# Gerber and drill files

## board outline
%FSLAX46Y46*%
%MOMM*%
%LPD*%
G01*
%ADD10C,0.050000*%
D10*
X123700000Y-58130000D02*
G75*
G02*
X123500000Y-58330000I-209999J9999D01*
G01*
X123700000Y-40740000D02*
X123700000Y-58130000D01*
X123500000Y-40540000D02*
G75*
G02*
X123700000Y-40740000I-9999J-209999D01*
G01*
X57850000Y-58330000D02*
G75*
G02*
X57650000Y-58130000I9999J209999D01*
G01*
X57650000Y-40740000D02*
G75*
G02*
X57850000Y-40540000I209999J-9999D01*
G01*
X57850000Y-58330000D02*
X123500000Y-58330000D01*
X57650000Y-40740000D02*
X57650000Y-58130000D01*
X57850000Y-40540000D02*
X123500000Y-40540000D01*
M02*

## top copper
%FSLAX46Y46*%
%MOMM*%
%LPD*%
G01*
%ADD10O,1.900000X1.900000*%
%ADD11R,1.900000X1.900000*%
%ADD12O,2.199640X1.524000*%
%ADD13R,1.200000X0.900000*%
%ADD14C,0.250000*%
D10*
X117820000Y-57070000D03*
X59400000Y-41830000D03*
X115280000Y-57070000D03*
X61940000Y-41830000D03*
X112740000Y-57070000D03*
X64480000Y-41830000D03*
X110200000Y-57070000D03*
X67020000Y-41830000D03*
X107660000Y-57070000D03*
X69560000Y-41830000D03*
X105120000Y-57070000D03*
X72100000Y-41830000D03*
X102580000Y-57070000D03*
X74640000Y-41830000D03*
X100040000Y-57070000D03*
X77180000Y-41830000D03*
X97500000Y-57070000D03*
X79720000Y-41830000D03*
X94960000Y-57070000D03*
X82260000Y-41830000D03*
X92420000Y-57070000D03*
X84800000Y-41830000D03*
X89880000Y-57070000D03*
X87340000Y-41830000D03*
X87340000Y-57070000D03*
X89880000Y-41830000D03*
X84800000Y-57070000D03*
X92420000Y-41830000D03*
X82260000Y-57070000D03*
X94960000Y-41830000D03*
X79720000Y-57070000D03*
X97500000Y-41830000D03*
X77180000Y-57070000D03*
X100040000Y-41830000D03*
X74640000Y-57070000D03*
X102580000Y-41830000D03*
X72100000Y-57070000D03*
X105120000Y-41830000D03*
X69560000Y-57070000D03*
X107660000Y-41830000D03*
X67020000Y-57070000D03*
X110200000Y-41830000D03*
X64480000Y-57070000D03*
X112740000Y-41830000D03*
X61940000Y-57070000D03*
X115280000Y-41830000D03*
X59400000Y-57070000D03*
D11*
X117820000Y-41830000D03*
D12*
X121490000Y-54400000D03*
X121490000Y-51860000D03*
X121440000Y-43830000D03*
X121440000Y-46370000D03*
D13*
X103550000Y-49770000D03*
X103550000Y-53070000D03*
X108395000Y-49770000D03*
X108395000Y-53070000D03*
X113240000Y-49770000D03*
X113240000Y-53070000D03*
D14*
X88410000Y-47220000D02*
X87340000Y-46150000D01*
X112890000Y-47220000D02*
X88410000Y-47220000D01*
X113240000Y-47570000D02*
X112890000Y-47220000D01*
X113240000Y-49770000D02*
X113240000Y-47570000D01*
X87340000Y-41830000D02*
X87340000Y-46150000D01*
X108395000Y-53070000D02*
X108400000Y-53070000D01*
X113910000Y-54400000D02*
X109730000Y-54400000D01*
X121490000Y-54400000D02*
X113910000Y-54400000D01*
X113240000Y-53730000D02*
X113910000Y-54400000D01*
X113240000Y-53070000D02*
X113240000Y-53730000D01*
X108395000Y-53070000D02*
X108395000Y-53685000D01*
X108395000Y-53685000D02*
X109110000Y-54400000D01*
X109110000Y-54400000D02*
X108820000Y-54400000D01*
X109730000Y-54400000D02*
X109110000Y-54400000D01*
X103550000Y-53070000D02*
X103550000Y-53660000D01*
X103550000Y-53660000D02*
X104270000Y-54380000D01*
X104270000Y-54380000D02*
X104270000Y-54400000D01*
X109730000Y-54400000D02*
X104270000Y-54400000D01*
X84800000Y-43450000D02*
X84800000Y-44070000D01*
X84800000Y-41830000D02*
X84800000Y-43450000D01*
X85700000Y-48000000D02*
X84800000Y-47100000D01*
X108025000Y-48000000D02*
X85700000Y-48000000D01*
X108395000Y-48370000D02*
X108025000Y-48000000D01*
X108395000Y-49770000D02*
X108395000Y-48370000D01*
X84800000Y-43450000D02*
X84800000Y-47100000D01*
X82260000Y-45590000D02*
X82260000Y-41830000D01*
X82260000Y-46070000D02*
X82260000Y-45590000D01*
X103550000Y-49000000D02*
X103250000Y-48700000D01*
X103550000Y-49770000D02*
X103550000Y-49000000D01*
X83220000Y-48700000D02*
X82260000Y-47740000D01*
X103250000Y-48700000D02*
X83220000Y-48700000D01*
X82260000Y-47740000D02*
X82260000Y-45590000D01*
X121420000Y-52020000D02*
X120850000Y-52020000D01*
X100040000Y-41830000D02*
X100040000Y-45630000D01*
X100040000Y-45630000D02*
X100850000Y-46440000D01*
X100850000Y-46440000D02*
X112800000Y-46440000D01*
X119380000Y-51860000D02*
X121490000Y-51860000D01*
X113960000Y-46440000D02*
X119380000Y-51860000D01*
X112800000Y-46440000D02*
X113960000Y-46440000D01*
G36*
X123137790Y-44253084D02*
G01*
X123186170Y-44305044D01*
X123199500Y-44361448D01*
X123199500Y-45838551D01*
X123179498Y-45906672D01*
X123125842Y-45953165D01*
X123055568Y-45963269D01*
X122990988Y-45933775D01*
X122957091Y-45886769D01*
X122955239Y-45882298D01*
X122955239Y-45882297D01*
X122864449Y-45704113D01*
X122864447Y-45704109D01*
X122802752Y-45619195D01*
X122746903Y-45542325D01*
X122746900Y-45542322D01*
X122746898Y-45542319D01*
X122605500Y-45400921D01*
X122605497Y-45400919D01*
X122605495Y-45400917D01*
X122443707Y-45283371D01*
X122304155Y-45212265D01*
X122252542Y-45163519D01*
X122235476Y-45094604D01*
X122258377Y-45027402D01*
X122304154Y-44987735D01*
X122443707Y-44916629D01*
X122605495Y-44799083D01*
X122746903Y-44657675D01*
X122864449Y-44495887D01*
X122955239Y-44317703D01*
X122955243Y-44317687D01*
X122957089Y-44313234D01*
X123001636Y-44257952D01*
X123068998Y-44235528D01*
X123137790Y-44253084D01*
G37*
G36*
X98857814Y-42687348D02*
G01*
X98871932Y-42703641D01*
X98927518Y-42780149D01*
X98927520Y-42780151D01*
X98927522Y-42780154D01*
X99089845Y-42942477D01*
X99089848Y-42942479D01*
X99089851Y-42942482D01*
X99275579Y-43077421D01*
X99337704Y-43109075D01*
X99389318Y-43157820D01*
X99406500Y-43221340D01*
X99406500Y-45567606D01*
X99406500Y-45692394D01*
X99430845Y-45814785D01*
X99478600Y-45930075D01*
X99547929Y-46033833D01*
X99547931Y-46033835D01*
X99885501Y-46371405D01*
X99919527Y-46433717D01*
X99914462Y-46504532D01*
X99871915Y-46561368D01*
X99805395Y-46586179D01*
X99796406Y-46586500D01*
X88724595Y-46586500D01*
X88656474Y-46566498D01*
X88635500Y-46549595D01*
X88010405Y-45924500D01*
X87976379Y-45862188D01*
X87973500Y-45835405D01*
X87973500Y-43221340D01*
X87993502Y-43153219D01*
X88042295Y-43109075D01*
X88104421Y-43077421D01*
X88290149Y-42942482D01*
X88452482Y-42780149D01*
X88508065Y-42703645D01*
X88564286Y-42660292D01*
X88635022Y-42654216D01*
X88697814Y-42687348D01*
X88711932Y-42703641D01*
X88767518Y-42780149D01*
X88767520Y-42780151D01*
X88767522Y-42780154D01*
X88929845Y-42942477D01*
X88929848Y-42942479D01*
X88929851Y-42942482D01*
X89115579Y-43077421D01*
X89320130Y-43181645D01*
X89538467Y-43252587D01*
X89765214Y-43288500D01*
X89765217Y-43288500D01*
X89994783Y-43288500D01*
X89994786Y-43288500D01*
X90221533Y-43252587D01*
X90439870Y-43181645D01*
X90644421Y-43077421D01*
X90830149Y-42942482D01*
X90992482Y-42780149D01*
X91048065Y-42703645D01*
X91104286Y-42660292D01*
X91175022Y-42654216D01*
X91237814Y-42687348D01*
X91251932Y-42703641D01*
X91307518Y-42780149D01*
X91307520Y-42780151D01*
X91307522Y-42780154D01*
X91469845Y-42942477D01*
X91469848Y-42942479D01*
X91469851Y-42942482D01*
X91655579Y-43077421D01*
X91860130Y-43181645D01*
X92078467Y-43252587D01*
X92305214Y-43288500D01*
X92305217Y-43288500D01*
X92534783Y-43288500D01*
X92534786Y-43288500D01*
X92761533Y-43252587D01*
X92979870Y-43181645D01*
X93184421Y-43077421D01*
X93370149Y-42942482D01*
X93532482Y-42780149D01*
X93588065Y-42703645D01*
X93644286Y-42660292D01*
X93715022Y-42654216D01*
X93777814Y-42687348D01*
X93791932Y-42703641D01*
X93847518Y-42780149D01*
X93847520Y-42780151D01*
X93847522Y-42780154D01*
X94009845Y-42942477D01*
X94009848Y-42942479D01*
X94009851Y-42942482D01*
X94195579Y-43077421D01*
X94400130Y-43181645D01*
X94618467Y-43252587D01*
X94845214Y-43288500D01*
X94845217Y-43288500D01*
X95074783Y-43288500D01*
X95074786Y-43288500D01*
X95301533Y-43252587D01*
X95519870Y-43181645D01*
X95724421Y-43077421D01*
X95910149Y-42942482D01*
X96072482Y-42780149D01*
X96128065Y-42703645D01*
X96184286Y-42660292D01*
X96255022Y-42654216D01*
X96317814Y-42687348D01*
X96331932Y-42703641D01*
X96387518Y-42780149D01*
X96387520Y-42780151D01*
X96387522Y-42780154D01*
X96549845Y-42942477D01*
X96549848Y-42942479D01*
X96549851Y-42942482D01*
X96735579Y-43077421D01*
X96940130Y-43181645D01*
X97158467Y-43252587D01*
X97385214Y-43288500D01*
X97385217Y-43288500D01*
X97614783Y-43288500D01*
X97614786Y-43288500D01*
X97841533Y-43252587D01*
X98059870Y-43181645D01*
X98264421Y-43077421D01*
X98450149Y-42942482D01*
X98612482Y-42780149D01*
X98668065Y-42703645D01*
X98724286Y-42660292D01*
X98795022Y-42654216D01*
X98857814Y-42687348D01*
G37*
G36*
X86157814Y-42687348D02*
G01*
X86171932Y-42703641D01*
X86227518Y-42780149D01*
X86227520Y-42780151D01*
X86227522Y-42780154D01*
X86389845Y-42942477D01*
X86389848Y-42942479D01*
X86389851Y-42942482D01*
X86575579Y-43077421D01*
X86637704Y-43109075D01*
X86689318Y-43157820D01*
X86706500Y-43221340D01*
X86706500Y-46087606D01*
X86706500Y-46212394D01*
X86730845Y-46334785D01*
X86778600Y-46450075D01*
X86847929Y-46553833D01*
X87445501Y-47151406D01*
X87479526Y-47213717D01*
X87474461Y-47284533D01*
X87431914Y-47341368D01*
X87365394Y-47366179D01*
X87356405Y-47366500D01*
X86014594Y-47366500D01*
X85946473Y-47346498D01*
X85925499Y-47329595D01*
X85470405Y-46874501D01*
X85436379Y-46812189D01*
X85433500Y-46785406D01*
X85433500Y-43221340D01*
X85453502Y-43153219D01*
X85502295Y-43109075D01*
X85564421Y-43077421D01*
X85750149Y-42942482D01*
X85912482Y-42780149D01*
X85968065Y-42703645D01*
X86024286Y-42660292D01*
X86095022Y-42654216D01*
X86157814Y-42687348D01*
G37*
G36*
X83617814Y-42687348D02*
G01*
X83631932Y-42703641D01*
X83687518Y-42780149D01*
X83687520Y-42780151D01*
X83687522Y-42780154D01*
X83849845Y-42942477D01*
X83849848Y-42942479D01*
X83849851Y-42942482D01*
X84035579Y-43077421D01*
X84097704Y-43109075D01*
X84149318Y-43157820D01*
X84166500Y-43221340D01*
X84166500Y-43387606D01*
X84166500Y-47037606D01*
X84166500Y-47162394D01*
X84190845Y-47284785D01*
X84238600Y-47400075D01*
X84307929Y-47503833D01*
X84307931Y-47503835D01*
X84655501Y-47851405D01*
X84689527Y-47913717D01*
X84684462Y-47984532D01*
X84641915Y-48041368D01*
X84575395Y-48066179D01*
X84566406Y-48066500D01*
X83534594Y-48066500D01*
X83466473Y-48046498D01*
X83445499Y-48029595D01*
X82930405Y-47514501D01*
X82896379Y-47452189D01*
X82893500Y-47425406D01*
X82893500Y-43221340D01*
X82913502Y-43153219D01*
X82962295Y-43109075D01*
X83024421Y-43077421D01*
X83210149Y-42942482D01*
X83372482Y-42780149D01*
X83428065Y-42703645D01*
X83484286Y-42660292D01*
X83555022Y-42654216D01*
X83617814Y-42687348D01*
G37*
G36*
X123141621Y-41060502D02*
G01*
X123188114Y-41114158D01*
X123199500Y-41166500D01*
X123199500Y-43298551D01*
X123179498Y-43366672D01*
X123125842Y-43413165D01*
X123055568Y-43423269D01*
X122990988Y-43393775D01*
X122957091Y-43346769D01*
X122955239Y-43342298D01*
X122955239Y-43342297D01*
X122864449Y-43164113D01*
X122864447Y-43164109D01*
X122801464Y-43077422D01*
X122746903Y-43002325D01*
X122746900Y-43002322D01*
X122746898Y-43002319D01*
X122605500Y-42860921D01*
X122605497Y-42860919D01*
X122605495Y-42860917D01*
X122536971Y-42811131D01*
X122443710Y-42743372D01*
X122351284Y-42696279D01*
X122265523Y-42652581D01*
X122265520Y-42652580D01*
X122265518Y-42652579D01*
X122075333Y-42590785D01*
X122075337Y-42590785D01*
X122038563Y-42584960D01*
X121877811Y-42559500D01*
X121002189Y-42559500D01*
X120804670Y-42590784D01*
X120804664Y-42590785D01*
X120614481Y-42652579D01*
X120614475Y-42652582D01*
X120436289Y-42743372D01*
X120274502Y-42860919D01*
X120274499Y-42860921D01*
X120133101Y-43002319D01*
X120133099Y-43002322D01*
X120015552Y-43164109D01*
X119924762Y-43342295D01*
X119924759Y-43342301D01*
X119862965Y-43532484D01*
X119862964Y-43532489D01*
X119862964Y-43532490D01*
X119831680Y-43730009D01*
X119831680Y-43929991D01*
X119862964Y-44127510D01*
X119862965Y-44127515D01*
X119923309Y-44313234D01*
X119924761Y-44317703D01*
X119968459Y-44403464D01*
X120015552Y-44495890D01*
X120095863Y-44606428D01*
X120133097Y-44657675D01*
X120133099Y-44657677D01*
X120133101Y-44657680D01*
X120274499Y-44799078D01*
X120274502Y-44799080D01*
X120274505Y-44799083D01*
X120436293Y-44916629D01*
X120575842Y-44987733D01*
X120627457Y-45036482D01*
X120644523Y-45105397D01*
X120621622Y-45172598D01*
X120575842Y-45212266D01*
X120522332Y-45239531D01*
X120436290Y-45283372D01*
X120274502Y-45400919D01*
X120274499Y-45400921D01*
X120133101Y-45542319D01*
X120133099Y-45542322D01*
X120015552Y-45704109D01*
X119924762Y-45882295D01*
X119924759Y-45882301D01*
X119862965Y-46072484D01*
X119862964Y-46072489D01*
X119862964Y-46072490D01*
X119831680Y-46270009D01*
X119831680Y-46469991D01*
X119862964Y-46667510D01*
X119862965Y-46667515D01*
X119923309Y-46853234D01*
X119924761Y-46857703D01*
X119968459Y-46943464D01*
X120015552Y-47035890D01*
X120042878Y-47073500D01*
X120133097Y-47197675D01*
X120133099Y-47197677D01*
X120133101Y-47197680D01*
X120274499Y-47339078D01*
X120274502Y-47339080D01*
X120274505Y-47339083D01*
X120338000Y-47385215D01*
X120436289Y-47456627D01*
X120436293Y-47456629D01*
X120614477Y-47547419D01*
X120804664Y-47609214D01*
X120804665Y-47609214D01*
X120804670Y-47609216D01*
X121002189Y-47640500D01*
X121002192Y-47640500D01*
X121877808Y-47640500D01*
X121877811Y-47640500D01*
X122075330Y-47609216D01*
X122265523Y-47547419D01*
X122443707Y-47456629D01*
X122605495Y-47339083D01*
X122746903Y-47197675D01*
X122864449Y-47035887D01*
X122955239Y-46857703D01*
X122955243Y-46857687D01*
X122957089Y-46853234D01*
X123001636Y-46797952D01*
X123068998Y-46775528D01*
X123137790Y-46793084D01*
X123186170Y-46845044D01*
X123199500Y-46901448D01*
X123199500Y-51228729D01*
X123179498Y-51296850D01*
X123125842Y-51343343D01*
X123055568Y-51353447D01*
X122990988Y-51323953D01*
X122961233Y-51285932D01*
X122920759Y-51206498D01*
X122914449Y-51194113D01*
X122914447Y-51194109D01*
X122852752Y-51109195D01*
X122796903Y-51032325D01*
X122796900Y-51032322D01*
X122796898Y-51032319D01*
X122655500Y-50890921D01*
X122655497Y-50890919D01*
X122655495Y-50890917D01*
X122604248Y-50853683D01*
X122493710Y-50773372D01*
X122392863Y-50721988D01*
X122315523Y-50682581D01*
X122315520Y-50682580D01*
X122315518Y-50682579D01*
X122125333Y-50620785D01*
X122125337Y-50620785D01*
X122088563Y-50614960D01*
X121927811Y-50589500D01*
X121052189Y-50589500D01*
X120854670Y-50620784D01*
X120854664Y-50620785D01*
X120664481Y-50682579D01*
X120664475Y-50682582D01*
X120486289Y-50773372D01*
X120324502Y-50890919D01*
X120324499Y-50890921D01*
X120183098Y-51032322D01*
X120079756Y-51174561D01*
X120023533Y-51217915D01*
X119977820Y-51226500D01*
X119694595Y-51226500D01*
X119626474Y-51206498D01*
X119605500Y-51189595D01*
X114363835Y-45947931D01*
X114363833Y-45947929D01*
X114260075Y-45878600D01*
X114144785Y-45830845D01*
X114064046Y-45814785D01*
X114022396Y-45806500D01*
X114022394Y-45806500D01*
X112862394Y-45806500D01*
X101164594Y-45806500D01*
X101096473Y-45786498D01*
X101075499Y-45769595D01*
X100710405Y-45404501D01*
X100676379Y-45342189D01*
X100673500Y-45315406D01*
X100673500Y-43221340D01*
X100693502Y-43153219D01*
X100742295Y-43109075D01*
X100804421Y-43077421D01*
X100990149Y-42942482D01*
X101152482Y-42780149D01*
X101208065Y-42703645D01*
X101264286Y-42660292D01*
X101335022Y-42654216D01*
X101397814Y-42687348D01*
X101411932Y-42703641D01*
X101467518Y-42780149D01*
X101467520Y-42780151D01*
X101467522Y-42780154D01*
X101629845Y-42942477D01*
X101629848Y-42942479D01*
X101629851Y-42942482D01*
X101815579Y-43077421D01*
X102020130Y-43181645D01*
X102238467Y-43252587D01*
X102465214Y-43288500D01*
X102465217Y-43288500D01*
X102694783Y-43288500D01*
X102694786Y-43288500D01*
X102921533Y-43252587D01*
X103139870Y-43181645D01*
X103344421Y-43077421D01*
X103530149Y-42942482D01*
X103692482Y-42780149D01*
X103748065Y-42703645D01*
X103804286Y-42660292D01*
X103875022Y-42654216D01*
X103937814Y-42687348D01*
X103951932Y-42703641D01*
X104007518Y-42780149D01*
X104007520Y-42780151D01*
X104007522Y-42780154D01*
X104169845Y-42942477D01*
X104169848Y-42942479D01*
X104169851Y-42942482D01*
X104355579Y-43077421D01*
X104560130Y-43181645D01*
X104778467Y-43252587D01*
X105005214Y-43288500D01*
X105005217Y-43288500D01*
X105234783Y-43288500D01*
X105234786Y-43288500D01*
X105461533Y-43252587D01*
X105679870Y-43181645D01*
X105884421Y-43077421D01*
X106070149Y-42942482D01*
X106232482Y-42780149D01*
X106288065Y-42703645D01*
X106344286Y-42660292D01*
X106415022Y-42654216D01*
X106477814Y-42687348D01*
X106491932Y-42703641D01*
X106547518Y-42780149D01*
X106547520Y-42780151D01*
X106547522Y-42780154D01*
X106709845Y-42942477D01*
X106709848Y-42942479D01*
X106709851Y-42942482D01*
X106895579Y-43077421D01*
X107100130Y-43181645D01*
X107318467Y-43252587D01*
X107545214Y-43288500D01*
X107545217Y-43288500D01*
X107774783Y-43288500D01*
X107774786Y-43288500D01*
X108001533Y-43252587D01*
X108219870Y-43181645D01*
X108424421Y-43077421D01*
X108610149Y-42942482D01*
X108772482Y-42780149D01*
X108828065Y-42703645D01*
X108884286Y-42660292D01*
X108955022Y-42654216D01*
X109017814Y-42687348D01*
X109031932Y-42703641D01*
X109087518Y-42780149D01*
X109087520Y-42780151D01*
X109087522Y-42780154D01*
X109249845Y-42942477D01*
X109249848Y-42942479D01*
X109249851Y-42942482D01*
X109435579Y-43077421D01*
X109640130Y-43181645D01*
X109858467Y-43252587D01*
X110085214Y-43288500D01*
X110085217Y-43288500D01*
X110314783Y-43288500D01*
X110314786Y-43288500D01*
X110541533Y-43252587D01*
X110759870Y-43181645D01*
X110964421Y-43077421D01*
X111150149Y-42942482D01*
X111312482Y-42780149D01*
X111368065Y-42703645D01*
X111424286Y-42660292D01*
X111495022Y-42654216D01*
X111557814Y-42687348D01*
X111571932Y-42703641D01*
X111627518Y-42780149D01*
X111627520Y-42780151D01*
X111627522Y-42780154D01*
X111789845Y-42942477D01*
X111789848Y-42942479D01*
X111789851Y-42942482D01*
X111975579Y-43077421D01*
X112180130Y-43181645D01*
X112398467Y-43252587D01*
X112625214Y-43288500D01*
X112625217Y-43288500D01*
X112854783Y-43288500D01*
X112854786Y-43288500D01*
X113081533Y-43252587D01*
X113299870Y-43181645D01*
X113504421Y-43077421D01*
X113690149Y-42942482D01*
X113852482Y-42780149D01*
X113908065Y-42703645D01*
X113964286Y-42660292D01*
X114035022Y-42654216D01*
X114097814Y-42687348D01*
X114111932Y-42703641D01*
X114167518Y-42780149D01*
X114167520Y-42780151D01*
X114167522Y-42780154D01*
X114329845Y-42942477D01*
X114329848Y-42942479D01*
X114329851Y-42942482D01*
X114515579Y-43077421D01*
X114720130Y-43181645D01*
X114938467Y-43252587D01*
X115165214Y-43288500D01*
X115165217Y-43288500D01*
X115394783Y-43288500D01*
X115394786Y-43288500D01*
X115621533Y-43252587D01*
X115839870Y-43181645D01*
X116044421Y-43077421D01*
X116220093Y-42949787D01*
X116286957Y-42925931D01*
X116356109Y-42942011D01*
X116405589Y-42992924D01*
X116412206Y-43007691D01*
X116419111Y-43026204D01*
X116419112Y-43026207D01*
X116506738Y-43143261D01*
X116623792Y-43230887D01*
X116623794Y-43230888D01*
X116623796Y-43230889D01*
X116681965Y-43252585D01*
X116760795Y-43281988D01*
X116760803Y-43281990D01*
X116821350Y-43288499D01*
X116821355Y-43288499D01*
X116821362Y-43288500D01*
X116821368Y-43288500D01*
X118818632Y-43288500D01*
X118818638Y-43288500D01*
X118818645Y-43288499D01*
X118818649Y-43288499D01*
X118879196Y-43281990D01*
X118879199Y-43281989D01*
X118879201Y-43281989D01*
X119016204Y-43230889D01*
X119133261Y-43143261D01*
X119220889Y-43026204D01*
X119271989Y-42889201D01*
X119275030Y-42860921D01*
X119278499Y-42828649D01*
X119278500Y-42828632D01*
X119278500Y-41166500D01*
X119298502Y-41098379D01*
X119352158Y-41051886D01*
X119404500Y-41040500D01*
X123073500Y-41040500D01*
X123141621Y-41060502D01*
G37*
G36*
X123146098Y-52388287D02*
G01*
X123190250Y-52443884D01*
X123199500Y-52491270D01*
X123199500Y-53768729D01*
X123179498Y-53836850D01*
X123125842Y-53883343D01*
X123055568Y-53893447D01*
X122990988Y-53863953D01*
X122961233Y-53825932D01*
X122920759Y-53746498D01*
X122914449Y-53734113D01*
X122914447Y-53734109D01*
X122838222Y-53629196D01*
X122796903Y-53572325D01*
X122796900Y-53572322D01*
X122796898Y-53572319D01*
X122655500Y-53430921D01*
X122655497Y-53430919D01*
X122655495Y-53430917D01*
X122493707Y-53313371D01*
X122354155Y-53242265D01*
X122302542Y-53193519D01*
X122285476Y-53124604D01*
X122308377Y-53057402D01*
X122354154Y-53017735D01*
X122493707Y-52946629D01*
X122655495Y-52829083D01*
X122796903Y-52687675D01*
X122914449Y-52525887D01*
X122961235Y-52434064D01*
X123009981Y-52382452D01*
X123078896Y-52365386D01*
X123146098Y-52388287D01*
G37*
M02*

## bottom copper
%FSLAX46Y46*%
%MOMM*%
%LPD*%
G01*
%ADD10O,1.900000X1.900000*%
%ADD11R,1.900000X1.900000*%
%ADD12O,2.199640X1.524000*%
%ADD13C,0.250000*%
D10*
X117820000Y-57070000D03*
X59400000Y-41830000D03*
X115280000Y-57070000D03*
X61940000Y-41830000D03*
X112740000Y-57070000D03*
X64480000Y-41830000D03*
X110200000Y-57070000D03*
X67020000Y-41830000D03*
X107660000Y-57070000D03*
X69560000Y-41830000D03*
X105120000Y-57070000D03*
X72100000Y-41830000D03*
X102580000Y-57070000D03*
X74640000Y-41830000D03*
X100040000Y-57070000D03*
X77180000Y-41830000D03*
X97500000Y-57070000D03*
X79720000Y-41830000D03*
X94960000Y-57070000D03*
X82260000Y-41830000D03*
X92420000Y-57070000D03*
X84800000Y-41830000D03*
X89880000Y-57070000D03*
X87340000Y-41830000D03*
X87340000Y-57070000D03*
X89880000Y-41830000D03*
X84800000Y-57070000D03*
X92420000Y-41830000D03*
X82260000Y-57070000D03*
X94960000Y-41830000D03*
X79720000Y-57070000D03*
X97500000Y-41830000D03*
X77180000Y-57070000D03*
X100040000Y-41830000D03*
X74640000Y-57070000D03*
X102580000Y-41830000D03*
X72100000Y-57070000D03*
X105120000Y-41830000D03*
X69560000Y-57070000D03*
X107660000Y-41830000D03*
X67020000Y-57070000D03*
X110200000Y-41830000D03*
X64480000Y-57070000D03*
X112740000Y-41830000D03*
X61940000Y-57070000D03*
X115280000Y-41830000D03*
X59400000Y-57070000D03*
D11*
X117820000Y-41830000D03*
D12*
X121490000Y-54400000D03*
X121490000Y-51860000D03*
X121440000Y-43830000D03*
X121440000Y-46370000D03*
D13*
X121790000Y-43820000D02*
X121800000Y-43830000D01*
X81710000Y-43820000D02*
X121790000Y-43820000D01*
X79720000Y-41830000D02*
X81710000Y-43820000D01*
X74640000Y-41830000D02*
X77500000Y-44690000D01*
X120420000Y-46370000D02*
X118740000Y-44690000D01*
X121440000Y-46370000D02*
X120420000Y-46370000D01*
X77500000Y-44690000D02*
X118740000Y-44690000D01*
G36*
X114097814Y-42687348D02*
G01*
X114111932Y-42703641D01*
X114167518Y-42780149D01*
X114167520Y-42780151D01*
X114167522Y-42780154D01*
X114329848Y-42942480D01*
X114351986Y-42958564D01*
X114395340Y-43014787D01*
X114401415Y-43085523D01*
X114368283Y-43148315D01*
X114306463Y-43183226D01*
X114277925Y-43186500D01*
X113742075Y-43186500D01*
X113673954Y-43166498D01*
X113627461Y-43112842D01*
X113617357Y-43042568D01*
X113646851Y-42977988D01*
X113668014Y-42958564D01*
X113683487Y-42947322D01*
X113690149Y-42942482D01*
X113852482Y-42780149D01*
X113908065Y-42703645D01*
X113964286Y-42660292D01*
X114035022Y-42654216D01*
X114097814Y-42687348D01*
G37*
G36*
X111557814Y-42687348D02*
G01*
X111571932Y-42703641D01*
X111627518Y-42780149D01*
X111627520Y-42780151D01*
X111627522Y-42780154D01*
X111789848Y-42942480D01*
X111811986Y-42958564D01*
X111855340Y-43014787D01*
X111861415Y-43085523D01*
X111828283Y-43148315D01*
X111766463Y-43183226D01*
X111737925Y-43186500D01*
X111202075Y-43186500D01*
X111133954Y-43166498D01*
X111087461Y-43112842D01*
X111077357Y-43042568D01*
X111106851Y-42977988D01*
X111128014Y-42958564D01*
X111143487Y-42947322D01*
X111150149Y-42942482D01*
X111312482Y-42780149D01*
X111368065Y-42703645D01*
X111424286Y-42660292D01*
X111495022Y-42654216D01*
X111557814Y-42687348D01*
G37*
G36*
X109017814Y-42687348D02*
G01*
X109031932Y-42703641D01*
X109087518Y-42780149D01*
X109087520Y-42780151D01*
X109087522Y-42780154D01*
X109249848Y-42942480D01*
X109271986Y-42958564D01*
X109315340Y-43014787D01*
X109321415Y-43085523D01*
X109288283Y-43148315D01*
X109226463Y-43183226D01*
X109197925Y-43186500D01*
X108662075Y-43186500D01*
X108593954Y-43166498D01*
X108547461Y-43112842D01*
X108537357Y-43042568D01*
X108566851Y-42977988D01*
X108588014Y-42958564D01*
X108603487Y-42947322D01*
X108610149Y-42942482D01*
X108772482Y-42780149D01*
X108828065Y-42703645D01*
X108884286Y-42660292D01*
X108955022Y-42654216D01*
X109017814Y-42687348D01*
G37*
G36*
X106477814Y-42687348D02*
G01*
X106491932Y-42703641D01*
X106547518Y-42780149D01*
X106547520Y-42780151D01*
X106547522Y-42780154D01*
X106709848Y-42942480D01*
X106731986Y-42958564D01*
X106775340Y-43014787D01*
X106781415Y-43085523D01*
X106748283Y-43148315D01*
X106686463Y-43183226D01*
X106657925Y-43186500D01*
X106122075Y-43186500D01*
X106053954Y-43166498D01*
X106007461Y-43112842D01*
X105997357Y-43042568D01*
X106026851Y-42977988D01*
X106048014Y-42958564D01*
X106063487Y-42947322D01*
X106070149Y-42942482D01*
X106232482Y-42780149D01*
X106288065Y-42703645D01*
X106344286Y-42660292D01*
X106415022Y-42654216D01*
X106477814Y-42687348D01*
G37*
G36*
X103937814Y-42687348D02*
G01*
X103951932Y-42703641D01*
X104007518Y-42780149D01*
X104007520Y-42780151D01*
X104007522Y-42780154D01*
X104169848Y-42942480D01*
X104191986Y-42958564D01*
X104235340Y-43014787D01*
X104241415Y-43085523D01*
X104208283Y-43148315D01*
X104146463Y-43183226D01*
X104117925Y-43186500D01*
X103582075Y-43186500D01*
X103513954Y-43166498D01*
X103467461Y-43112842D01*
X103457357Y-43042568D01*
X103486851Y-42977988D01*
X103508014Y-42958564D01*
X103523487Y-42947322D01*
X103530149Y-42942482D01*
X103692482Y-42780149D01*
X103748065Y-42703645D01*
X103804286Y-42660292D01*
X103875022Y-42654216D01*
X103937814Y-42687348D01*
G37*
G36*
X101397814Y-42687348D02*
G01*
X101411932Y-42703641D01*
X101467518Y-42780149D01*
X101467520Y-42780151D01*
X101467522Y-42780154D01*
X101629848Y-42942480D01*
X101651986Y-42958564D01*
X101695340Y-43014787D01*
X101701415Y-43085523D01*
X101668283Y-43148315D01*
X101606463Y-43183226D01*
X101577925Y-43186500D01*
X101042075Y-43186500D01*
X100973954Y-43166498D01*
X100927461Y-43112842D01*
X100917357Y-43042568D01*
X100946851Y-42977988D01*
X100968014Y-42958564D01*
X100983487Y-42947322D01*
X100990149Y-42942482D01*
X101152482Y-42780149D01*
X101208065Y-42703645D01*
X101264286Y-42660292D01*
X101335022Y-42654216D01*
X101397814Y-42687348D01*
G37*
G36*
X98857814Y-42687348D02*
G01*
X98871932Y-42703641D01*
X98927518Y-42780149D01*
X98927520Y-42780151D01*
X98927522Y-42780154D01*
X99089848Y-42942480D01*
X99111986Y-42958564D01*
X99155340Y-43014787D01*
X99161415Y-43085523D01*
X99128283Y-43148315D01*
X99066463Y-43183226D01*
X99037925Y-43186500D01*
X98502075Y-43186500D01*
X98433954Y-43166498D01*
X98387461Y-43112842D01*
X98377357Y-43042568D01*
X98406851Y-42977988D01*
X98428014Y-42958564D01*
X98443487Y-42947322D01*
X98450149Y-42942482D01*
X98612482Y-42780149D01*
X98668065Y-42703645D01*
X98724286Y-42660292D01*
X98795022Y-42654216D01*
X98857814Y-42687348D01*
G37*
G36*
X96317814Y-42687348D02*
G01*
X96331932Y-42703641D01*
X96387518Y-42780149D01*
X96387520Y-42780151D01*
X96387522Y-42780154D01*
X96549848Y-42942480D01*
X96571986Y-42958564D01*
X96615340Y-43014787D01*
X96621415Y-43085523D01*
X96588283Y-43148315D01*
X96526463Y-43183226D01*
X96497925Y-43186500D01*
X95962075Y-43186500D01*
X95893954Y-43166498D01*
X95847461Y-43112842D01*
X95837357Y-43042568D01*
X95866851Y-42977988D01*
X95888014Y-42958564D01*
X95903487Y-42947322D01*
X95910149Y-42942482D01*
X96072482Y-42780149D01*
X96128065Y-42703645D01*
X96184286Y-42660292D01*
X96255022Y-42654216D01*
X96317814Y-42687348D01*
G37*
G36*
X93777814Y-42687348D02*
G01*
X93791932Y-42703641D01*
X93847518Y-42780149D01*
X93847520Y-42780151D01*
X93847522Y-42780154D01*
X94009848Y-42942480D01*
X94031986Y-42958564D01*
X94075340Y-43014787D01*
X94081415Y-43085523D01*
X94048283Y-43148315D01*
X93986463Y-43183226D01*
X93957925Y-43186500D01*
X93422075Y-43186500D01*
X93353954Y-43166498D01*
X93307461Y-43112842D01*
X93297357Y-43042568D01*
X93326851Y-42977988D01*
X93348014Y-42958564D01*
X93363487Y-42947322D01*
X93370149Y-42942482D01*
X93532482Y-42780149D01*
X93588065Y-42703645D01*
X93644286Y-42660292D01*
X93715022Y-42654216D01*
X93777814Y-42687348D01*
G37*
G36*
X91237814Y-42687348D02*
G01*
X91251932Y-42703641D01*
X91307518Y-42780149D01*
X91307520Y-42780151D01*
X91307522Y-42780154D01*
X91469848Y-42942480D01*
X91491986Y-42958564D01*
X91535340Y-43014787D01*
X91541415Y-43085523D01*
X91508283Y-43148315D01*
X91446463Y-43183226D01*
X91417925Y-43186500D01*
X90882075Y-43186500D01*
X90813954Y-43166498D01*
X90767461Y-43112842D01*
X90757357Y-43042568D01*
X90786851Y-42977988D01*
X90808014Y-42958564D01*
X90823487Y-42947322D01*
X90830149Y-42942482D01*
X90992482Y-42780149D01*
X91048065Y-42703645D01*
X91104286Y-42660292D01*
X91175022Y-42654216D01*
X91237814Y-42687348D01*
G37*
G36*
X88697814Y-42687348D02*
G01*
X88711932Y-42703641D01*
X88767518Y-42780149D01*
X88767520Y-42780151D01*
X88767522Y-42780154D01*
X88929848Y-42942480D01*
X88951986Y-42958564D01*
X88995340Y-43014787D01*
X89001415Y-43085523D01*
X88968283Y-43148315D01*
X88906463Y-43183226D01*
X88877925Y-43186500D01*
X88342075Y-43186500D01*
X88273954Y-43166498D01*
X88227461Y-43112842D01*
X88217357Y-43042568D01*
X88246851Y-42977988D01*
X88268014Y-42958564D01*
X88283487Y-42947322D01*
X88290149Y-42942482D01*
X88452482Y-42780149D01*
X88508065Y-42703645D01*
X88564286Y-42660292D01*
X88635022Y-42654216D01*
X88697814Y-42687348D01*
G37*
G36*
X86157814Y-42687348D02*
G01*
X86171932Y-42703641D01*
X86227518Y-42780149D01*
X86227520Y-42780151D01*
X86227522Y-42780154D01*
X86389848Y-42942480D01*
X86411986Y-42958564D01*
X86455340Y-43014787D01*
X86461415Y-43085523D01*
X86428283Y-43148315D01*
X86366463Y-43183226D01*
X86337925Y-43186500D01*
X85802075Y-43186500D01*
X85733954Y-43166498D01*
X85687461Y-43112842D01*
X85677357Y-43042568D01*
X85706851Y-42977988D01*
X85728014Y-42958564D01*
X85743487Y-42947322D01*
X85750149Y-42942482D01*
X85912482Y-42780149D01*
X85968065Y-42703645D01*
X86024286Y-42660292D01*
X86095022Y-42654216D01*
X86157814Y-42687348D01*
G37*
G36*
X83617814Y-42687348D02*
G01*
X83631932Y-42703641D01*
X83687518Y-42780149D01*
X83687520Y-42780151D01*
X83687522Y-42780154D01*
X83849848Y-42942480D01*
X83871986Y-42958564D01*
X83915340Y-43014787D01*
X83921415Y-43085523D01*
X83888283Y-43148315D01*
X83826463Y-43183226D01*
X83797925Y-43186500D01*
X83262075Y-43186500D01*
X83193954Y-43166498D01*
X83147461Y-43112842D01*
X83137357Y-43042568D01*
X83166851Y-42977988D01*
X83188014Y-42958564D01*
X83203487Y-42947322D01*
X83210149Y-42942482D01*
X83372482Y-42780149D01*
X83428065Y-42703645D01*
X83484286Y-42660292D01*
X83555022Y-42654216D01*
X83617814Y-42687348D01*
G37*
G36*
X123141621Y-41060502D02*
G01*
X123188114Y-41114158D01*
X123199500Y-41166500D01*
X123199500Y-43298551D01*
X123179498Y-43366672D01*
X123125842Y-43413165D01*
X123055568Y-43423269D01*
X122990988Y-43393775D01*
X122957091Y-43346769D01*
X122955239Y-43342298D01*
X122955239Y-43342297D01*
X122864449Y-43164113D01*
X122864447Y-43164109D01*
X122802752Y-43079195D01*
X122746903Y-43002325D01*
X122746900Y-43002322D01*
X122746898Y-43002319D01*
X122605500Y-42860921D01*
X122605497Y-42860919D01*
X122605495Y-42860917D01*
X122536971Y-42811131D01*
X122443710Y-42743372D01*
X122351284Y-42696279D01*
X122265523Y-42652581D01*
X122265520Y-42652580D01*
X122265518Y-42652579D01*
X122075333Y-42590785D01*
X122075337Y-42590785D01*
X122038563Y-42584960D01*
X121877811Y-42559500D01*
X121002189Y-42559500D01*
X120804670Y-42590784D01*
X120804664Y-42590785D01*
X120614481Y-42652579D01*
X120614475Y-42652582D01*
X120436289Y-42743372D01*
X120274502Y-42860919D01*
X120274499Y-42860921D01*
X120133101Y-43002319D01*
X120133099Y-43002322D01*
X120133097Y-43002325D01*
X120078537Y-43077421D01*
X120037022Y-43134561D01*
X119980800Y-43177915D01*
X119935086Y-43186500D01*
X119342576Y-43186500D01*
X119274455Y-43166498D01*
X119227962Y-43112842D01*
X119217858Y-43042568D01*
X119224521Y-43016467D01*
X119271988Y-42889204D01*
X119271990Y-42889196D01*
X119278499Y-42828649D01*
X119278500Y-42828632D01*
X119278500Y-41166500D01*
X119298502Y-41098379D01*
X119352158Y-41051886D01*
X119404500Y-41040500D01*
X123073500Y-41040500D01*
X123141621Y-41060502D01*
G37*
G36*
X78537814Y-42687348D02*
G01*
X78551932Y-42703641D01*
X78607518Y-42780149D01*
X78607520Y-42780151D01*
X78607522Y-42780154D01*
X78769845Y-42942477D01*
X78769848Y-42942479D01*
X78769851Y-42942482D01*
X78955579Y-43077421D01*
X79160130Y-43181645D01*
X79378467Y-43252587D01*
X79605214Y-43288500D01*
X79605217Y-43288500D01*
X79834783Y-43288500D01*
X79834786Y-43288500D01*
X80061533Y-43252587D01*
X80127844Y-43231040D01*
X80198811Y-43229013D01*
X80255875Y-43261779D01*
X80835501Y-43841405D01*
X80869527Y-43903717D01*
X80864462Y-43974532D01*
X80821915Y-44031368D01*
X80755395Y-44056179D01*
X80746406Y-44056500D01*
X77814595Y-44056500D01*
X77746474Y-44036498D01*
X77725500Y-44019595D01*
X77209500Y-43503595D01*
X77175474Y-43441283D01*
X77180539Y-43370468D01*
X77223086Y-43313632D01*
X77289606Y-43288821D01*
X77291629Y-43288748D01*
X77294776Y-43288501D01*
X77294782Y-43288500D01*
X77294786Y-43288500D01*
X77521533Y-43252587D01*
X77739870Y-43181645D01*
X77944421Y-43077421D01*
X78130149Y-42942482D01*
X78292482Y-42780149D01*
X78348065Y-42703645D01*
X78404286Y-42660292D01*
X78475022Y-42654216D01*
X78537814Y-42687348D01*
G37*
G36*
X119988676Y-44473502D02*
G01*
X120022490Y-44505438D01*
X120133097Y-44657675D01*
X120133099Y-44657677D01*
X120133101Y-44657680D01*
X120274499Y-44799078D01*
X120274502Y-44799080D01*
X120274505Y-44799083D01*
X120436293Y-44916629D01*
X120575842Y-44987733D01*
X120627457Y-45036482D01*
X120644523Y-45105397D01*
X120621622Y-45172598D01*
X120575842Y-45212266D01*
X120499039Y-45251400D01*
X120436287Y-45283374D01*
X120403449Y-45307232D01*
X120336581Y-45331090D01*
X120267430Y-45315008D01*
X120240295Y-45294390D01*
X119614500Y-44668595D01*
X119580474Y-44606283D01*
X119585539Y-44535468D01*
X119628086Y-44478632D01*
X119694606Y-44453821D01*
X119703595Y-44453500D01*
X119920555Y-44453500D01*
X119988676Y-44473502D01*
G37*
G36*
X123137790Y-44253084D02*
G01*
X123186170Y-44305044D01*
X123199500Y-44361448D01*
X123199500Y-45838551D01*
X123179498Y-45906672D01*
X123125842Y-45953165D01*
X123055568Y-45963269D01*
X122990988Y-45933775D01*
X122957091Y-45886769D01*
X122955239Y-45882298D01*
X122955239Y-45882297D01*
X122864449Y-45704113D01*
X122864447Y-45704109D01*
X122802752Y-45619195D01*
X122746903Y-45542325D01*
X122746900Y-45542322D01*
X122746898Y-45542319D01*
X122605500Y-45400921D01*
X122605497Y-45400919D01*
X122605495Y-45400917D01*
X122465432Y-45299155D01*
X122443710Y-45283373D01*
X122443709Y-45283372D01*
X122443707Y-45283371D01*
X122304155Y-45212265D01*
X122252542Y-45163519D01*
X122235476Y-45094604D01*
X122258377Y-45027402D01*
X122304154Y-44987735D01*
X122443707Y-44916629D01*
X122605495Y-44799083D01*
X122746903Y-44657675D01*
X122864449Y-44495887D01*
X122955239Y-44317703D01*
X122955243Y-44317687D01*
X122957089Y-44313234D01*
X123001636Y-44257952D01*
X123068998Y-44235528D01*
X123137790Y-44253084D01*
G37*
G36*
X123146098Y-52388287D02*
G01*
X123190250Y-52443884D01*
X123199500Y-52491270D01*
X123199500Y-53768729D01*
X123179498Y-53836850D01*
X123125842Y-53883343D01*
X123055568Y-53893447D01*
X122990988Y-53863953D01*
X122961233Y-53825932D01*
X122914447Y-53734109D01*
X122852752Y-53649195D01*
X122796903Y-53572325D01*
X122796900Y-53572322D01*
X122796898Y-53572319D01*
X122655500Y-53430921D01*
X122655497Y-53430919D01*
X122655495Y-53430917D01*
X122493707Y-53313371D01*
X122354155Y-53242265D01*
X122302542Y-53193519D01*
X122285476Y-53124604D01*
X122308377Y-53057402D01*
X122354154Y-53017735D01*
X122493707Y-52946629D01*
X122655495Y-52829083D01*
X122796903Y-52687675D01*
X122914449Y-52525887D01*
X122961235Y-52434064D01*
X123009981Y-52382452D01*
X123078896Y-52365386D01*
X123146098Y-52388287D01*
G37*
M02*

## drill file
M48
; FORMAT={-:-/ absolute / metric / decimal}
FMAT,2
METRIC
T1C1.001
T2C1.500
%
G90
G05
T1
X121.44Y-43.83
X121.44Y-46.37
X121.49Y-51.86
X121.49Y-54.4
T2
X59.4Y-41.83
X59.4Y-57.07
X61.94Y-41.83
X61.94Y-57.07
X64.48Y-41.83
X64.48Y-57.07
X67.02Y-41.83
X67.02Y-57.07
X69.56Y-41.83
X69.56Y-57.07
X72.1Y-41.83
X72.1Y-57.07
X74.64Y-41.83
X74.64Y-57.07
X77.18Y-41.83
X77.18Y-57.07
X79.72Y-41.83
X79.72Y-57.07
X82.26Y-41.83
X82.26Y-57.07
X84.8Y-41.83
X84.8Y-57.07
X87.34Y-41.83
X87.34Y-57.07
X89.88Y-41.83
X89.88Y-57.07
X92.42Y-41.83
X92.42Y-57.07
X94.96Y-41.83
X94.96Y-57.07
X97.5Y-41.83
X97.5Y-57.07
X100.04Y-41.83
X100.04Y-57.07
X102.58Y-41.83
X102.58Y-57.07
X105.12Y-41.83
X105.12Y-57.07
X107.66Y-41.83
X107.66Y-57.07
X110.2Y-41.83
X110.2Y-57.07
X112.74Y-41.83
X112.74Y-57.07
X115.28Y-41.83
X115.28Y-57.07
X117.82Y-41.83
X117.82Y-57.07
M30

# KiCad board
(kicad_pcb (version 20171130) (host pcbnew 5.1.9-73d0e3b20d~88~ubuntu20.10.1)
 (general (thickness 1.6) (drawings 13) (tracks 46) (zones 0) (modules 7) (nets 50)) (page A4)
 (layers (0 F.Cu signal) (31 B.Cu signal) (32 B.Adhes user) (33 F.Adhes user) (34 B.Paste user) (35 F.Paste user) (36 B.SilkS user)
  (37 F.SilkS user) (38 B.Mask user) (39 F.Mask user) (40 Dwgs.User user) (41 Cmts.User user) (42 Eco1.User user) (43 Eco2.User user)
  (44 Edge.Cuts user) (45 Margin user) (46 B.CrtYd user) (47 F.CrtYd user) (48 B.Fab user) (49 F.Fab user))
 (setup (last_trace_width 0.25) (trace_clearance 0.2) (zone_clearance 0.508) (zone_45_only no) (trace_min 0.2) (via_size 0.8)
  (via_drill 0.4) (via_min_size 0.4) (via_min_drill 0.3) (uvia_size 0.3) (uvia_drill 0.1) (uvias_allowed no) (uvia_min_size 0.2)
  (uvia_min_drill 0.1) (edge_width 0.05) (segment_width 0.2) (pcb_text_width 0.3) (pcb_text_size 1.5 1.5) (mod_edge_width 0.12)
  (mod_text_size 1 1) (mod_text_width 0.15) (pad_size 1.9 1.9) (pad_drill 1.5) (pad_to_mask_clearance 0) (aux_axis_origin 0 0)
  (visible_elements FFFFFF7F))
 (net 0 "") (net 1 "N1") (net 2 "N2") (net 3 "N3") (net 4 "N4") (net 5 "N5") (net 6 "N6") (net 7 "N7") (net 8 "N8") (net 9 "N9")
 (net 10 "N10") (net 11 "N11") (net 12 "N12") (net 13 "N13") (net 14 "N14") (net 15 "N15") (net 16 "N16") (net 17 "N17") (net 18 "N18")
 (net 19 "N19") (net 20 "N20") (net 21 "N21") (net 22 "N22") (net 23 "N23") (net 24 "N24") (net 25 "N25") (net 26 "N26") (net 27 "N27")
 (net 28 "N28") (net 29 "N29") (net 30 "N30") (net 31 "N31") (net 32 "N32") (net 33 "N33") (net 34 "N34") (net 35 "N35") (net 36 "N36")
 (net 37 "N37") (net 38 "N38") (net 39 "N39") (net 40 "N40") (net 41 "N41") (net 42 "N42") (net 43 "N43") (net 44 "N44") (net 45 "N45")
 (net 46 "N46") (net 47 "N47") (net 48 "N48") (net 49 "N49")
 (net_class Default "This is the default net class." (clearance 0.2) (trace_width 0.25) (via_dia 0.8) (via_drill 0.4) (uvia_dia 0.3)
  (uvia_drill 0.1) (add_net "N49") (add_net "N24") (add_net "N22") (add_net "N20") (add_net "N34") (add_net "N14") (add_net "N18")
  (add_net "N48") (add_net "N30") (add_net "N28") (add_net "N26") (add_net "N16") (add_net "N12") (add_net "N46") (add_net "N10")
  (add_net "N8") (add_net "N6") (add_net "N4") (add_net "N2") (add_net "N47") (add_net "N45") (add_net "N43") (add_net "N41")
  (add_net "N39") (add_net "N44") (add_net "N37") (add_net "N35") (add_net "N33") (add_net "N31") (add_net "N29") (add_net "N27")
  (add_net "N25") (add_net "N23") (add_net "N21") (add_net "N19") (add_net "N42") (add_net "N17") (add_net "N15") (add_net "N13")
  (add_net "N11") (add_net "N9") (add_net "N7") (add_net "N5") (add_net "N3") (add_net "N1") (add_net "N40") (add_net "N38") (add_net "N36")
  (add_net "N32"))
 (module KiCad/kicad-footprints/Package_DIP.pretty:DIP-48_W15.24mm (layer F.Cu) (at 117.82 41.83 270)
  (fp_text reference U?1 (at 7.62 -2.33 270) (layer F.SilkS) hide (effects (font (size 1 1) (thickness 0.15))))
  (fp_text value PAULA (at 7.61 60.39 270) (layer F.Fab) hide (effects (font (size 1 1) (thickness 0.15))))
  (pad 48 thru_hole oval (at 15.24 0 270) (size 1.9 1.9) (drill 1.5) (layers *.Cu *.Mask) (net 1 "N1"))
  (pad 24 thru_hole oval (at 0 58.42 270) (size 1.9 1.9) (drill 1.5) (layers *.Cu *.Mask) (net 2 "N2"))
  (pad 47 thru_hole oval (at 15.24 2.54 270) (size 1.9 1.9) (drill 1.5) (layers *.Cu *.Mask) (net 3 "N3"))
  (pad 23 thru_hole oval (at 0 55.88 270) (size 1.9 1.9) (drill 1.5) (layers *.Cu *.Mask) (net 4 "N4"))
  (pad 46 thru_hole oval (at 15.24 5.08 270) (size 1.9 1.9) (drill 1.5) (layers *.Cu *.Mask) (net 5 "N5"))
  (pad 22 thru_hole oval (at 0 53.34 270) (size 1.9 1.9) (drill 1.5) (layers *.Cu *.Mask) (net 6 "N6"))
  (pad 45 thru_hole oval (at 15.24 7.62 270) (size 1.9 1.9) (drill 1.5) (layers *.Cu *.Mask) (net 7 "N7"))
  (pad 21 thru_hole oval (at 0 50.8 270) (size 1.9 1.9) (drill 1.5) (layers *.Cu *.Mask) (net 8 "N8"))
  (pad 44 thru_hole oval (at 15.24 10.16 270) (size 1.9 1.9) (drill 1.5) (layers *.Cu *.Mask) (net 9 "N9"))
  (pad 20 thru_hole oval (at 0 48.26 270) (size 1.9 1.9) (drill 1.5) (layers *.Cu *.Mask) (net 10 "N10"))
  (pad 43 thru_hole oval (at 15.24 12.7 270) (size 1.9 1.9) (drill 1.5) (layers *.Cu *.Mask) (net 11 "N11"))
  (pad 19 thru_hole oval (at 0 45.72 270) (size 1.9 1.9) (drill 1.5) (layers *.Cu *.Mask) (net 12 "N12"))
  (pad 42 thru_hole oval (at 15.24 15.24 270) (size 1.9 1.9) (drill 1.5) (layers *.Cu *.Mask) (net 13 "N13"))
  (pad 18 thru_hole oval (at 0 43.18 270) (size 1.9 1.9) (drill 1.5) (layers *.Cu *.Mask) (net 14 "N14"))
  (pad 41 thru_hole oval (at 15.24 17.78 270) (size 1.9 1.9) (drill 1.5) (layers *.Cu *.Mask) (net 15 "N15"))
  (pad 17 thru_hole oval (at 0 40.64 270) (size 1.9 1.9) (drill 1.5) (layers *.Cu *.Mask) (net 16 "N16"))
  (pad 40 thru_hole oval (at 15.24 20.32 270) (size 1.9 1.9) (drill 1.5) (layers *.Cu *.Mask) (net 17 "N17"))
  (pad 16 thru_hole oval (at 0 38.1 270) (size 1.9 1.9) (drill 1.5) (layers *.Cu *.Mask) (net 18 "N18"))
  (pad 39 thru_hole oval (at 15.24 22.86 270) (size 1.9 1.9) (drill 1.5) (layers *.Cu *.Mask) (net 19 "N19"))
  (pad 15 thru_hole oval (at 0 35.56 270) (size 1.9 1.9) (drill 1.5) (layers *.Cu *.Mask) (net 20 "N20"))
  (pad 38 thru_hole oval (at 15.24 25.4 270) (size 1.9 1.9) (drill 1.5) (layers *.Cu *.Mask) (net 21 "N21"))
  (pad 14 thru_hole oval (at 0 33.02 270) (size 1.9 1.9) (drill 1.5) (layers *.Cu *.Mask) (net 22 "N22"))
  (pad 37 thru_hole oval (at 15.24 27.94 270) (size 1.9 1.9) (drill 1.5) (layers *.Cu *.Mask) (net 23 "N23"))
  (pad 13 thru_hole oval (at 0 30.48 270) (size 1.9 1.9) (drill 1.5) (layers *.Cu *.Mask) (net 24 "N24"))
  (pad 36 thru_hole oval (at 15.24 30.48 270) (size 1.9 1.9) (drill 1.5) (layers *.Cu *.Mask) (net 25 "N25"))
  (pad 12 thru_hole oval (at 0 27.94 270) (size 1.9 1.9) (drill 1.5) (layers *.Cu *.Mask) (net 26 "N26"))
  (pad 35 thru_hole oval (at 15.24 33.02 270) (size 1.9 1.9) (drill 1.5) (layers *.Cu *.Mask) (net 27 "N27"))
  (pad 11 thru_hole oval (at 0 25.4 270) (size 1.9 1.9) (drill 1.5) (layers *.Cu *.Mask) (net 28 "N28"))
  (pad 34 thru_hole oval (at 15.24 35.56 270) (size 1.9 1.9) (drill 1.5) (layers *.Cu *.Mask) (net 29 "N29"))
  (pad 10 thru_hole oval (at 0 22.86 270) (size 1.9 1.9) (drill 1.5) (layers *.Cu *.Mask) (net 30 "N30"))
  (pad 33 thru_hole oval (at 15.24 38.1 270) (size 1.9 1.9) (drill 1.5) (layers *.Cu *.Mask) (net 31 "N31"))
  (pad 9 thru_hole oval (at 0 20.32 270) (size 1.9 1.9) (drill 1.5) (layers *.Cu *.Mask) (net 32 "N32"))
  (pad 32 thru_hole oval (at 15.24 40.64 270) (size 1.9 1.9) (drill 1.5) (layers *.Cu *.Mask) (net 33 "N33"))
  (pad 8 thru_hole oval (at 0 17.78 270) (size 1.9 1.9) (drill 1.5) (layers *.Cu *.Mask) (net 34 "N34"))
  (pad 31 thru_hole oval (at 15.24 43.18 270) (size 1.9 1.9) (drill 1.5) (layers *.Cu *.Mask) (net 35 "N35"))
  (pad 7 thru_hole oval (at 0 15.24 270) (size 1.9 1.9) (drill 1.5) (layers *.Cu *.Mask) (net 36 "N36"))
  (pad 30 thru_hole oval (at 15.24 45.72 270) (size 1.9 1.9) (drill 1.5) (layers *.Cu *.Mask) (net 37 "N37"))
  (pad 6 thru_hole oval (at 0 12.7 270) (size 1.9 1.9) (drill 1.5) (layers *.Cu *.Mask) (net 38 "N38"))
  (pad 29 thru_hole oval (at 15.24 48.26 270) (size 1.9 1.9) (drill 1.5) (layers *.Cu *.Mask) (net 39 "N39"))
  (pad 5 thru_hole oval (at 0 10.16 270) (size 1.9 1.9) (drill 1.5) (layers *.Cu *.Mask) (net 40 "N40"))
  (pad 28 thru_hole oval (at 15.24 50.8 270) (size 1.9 1.9) (drill 1.5) (layers *.Cu *.Mask) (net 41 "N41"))
  (pad 4 thru_hole oval (at 0 7.62 270) (size 1.9 1.9) (drill 1.5) (layers *.Cu *.Mask) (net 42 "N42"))
  (pad 27 thru_hole oval (at 15.24 53.34 270) (size 1.9 1.9) (drill 1.5) (layers *.Cu *.Mask) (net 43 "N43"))
  (pad 3 thru_hole oval (at 0 5.08 270) (size 1.9 1.9) (drill 1.5) (layers *.Cu *.Mask) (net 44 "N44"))
  (pad 26 thru_hole oval (at 15.24 55.88 270) (size 1.9 1.9) (drill 1.5) (layers *.Cu *.Mask) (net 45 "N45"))
  (pad 2 thru_hole oval (at 0 2.54 270) (size 1.9 1.9) (drill 1.5) (layers *.Cu *.Mask) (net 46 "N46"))
  (pad 25 thru_hole oval (at 15.24 58.42 270) (size 1.9 1.9) (drill 1.5) (layers *.Cu *.Mask) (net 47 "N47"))
  (pad 1 thru_hole rect (at 0 0 270) (size 1.9 1.9) (drill 1.5) (layers *.Cu *.Mask) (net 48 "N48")))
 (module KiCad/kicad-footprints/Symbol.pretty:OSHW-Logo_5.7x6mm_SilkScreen (layer F.Cu) (at 67 49.8 180)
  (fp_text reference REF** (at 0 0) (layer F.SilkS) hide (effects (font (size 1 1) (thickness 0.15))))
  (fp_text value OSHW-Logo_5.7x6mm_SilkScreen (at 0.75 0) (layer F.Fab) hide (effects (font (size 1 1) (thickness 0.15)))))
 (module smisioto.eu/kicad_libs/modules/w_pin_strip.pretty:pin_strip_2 (layer F.Cu) (at 121.49 53.13 270)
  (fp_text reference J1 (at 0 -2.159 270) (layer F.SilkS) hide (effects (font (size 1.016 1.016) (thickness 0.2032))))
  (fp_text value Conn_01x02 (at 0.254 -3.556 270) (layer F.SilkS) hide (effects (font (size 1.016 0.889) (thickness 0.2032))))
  (pad 2 thru_hole oval (at 1.27 0 270) (size 1.524 2.19964) (drill 1.00076) (layers *.Cu *.Mask F.SilkS) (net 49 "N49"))
  (pad 1 thru_hole oval (at -1.27 0 270) (size 1.524 2.19964) (drill 1.00076) (layers *.Cu *.Mask F.SilkS) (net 34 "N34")))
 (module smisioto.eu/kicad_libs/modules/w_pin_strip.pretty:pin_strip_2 (layer F.Cu) (at 121.44 45.1 90)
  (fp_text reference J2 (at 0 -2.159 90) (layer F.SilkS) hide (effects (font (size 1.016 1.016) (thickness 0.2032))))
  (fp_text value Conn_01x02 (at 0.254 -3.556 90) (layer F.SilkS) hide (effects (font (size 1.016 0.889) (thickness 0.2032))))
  (pad 2 thru_hole oval (at 1.27 0 90) (size 1.524 2.19964) (drill 1.00076) (layers *.Cu *.Mask F.SilkS) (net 18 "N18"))
  (pad 1 thru_hole oval (at -1.27 0 90) (size 1.524 2.19964) (drill 1.00076) (layers *.Cu *.Mask F.SilkS) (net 14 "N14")))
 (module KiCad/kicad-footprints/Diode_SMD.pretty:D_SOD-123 (layer F.Cu) (at 103.55 51.42 90)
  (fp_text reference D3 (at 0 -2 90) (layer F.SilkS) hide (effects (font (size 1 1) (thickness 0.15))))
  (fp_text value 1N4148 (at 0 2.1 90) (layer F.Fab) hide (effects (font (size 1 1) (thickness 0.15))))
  (pad 2 smd rect (at 1.65 0 90) (size 0.9 1.2) (layers F.Cu F.Paste F.Mask) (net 20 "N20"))
  (pad 1 smd rect (at -1.65 0 90) (size 0.9 1.2) (layers F.Cu F.Paste F.Mask) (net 49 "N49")))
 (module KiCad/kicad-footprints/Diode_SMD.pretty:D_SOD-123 (layer F.Cu) (at 108.395 51.42 90)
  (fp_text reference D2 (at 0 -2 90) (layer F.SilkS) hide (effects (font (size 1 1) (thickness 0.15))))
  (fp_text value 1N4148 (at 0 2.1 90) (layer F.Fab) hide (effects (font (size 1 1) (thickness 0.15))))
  (pad 2 smd rect (at 1.65 0 90) (size 0.9 1.2) (layers F.Cu F.Paste F.Mask) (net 22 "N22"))
  (pad 1 smd rect (at -1.65 0 90) (size 0.9 1.2) (layers F.Cu F.Paste F.Mask) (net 49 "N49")))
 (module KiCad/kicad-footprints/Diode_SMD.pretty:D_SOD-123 (layer F.Cu) (at 113.24 51.42 90)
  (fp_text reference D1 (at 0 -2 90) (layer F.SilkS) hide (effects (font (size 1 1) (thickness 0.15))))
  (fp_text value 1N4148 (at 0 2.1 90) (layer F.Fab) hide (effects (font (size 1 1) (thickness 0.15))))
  (pad 2 smd rect (at 1.65 0 90) (size 0.9 1.2) (layers F.Cu F.Paste F.Mask) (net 24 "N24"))
  (pad 1 smd rect (at -1.65 0 90) (size 0.9 1.2) (layers F.Cu F.Paste F.Mask) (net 49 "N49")))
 (gr_arc (start 123.490001 58.120001) (end 123.5 58.33) (angle -84.54789653) (layer Edge.Cuts) (width 0.05))
 (gr_line (start 123.7 40.74) (end 123.7 58.13) (layer Edge.Cuts) (width 0.05))
 (gr_arc (start 123.490001 40.749999) (end 123.7 40.74) (angle -84.54789653) (layer Edge.Cuts) (width 0.05))
 (gr_arc (start 57.859999 58.120001) (end 57.65 58.13) (angle -84.54789653) (layer Edge.Cuts) (width 0.05))
 (gr_arc (start 57.859999 40.749999) (end 57.85 40.54) (angle -84.54789653) (layer Edge.Cuts) (width 0.05))
 (gr_line (start 57.85 58.33) (end 123.5 58.33) (layer Edge.Cuts) (width 0.05))
 (gr_line (start 57.65 40.74) (end 57.65 58.13) (layer Edge.Cuts) (width 0.05))
 (gr_line (start 57.85 40.54) (end 123.5 40.54) (layer Edge.Cuts) (width 0.05))
 (segment (start 88.41 47.22) (end 87.34 46.15) (width 0.25) (layer F.Cu) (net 24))
 (segment (start 112.89 47.22) (end 88.41 47.22) (width 0.25) (layer F.Cu) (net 24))
 (segment (start 113.24 47.57) (end 112.89 47.22) (width 0.25) (layer F.Cu) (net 24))
 (segment (start 113.24 49.77) (end 113.24 47.57) (width 0.25) (layer F.Cu) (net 24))
 (segment (start 87.34 41.83) (end 87.34 46.15) (width 0.25) (layer F.Cu) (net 24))
 (segment (start 108.395 53.07) (end 108.4 53.07) (width 0.25) (layer F.Cu) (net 49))
 (segment (start 113.91 54.4) (end 109.73 54.4) (width 0.25) (layer F.Cu) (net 49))
 (segment (start 121.49 54.4) (end 113.91 54.4) (width 0.25) (layer F.Cu) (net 49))
 (segment (start 113.24 53.73) (end 113.91 54.4) (width 0.25) (layer F.Cu) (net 49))
 (segment (start 113.24 53.07) (end 113.24 53.73) (width 0.25) (layer F.Cu) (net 49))
 (segment (start 108.395 53.07) (end 108.395 53.685) (width 0.25) (layer F.Cu) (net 49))
 (segment (start 108.395 53.685) (end 109.11 54.4) (width 0.25) (layer F.Cu) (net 49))
 (segment (start 109.11 54.4) (end 108.82 54.4) (width 0.25) (layer F.Cu) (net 49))
 (segment (start 109.73 54.4) (end 109.11 54.4) (width 0.25) (layer F.Cu) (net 49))
 (segment (start 103.55 53.07) (end 103.55 53.66) (width 0.25) (layer F.Cu) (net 49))
 (segment (start 103.55 53.66) (end 104.27 54.38) (width 0.25) (layer F.Cu) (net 49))
 (segment (start 104.27 54.38) (end 104.27 54.4) (width 0.25) (layer F.Cu) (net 49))
 (segment (start 109.73 54.4) (end 104.27 54.4) (width 0.25) (layer F.Cu) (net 49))
 (segment (start 84.8 43.45) (end 84.8 44.07) (width 0.25) (layer F.Cu) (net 22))
 (segment (start 84.8 41.83) (end 84.8 43.45) (width 0.25) (layer F.Cu) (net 22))
 (segment (start 85.7 48) (end 84.8 47.1) (width 0.25) (layer F.Cu) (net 22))
 (segment (start 108.025 48) (end 85.7 48) (width 0.25) (layer F.Cu) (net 22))
 (segment (start 108.395 48.37) (end 108.025 48) (width 0.25) (layer F.Cu) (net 22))
 (segment (start 108.395 49.77) (end 108.395 48.37) (width 0.25) (layer F.Cu) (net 22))
 (segment (start 84.8 43.45) (end 84.8 47.1) (width 0.25) (layer F.Cu) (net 22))
 (segment (start 82.26 45.59) (end 82.26 41.83) (width 0.25) (layer F.Cu) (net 20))
 (segment (start 82.26 46.07) (end 82.26 45.59) (width 0.25) (layer F.Cu) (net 20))
 (segment (start 103.55 49) (end 103.25 48.7) (width 0.25) (layer F.Cu) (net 20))
 (segment (start 103.55 49.77) (end 103.55 49) (width 0.25) (layer F.Cu) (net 20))
 (segment (start 83.22 48.7) (end 82.26 47.74) (width 0.25) (layer F.Cu) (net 20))
 (segment (start 103.25 48.7) (end 83.22 48.7) (width 0.25) (layer F.Cu) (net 20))
 (segment (start 82.26 47.74) (end 82.26 45.59) (width 0.25) (layer F.Cu) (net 20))
 (segment (start 121.42 52.02) (end 120.85 52.02) (width 0.25) (layer F.Cu) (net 34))
 (segment (start 100.04 41.83) (end 100.04 45.63) (width 0.25) (layer F.Cu) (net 34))
 (segment (start 100.04 45.63) (end 100.85 46.44) (width 0.25) (layer F.Cu) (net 34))
 (segment (start 100.85 46.44) (end 112.8 46.44) (width 0.25) (layer F.Cu) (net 34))
 (segment (start 119.38 51.86) (end 121.49 51.86) (width 0.25) (layer F.Cu) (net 34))
 (segment (start 113.96 46.44) (end 119.38 51.86) (width 0.25) (layer F.Cu) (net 34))
 (segment (start 112.8 46.44) (end 113.96 46.44) (width 0.25) (layer F.Cu) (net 34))
 (segment (start 121.79 43.82) (end 121.8 43.83) (width 0.25) (layer B.Cu) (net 18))
 (segment (start 81.71 43.82) (end 121.79 43.82) (width 0.25) (layer B.Cu) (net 18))
 (segment (start 79.72 41.83) (end 81.71 43.82) (width 0.25) (layer B.Cu) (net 18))
 (segment (start 74.64 41.83) (end 77.5 44.69) (width 0.25) (layer B.Cu) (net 14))
 (segment (start 120.42 46.37) (end 118.74 44.69) (width 0.25) (layer B.Cu) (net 14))
 (segment (start 121.44 46.37) (end 120.42 46.37) (width 0.25) (layer B.Cu) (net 14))
 (segment (start 77.5 44.69) (end 118.74 44.69) (width 0.25) (layer B.Cu) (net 14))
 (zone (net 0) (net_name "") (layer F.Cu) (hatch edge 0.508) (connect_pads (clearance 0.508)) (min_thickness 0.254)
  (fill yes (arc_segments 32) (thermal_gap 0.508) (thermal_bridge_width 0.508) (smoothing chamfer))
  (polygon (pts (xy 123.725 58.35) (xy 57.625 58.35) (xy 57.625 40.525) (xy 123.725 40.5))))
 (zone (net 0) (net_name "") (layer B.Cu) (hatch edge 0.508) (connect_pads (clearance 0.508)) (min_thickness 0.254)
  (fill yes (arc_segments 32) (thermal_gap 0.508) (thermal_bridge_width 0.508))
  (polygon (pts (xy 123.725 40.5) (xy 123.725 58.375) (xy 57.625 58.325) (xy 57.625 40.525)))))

